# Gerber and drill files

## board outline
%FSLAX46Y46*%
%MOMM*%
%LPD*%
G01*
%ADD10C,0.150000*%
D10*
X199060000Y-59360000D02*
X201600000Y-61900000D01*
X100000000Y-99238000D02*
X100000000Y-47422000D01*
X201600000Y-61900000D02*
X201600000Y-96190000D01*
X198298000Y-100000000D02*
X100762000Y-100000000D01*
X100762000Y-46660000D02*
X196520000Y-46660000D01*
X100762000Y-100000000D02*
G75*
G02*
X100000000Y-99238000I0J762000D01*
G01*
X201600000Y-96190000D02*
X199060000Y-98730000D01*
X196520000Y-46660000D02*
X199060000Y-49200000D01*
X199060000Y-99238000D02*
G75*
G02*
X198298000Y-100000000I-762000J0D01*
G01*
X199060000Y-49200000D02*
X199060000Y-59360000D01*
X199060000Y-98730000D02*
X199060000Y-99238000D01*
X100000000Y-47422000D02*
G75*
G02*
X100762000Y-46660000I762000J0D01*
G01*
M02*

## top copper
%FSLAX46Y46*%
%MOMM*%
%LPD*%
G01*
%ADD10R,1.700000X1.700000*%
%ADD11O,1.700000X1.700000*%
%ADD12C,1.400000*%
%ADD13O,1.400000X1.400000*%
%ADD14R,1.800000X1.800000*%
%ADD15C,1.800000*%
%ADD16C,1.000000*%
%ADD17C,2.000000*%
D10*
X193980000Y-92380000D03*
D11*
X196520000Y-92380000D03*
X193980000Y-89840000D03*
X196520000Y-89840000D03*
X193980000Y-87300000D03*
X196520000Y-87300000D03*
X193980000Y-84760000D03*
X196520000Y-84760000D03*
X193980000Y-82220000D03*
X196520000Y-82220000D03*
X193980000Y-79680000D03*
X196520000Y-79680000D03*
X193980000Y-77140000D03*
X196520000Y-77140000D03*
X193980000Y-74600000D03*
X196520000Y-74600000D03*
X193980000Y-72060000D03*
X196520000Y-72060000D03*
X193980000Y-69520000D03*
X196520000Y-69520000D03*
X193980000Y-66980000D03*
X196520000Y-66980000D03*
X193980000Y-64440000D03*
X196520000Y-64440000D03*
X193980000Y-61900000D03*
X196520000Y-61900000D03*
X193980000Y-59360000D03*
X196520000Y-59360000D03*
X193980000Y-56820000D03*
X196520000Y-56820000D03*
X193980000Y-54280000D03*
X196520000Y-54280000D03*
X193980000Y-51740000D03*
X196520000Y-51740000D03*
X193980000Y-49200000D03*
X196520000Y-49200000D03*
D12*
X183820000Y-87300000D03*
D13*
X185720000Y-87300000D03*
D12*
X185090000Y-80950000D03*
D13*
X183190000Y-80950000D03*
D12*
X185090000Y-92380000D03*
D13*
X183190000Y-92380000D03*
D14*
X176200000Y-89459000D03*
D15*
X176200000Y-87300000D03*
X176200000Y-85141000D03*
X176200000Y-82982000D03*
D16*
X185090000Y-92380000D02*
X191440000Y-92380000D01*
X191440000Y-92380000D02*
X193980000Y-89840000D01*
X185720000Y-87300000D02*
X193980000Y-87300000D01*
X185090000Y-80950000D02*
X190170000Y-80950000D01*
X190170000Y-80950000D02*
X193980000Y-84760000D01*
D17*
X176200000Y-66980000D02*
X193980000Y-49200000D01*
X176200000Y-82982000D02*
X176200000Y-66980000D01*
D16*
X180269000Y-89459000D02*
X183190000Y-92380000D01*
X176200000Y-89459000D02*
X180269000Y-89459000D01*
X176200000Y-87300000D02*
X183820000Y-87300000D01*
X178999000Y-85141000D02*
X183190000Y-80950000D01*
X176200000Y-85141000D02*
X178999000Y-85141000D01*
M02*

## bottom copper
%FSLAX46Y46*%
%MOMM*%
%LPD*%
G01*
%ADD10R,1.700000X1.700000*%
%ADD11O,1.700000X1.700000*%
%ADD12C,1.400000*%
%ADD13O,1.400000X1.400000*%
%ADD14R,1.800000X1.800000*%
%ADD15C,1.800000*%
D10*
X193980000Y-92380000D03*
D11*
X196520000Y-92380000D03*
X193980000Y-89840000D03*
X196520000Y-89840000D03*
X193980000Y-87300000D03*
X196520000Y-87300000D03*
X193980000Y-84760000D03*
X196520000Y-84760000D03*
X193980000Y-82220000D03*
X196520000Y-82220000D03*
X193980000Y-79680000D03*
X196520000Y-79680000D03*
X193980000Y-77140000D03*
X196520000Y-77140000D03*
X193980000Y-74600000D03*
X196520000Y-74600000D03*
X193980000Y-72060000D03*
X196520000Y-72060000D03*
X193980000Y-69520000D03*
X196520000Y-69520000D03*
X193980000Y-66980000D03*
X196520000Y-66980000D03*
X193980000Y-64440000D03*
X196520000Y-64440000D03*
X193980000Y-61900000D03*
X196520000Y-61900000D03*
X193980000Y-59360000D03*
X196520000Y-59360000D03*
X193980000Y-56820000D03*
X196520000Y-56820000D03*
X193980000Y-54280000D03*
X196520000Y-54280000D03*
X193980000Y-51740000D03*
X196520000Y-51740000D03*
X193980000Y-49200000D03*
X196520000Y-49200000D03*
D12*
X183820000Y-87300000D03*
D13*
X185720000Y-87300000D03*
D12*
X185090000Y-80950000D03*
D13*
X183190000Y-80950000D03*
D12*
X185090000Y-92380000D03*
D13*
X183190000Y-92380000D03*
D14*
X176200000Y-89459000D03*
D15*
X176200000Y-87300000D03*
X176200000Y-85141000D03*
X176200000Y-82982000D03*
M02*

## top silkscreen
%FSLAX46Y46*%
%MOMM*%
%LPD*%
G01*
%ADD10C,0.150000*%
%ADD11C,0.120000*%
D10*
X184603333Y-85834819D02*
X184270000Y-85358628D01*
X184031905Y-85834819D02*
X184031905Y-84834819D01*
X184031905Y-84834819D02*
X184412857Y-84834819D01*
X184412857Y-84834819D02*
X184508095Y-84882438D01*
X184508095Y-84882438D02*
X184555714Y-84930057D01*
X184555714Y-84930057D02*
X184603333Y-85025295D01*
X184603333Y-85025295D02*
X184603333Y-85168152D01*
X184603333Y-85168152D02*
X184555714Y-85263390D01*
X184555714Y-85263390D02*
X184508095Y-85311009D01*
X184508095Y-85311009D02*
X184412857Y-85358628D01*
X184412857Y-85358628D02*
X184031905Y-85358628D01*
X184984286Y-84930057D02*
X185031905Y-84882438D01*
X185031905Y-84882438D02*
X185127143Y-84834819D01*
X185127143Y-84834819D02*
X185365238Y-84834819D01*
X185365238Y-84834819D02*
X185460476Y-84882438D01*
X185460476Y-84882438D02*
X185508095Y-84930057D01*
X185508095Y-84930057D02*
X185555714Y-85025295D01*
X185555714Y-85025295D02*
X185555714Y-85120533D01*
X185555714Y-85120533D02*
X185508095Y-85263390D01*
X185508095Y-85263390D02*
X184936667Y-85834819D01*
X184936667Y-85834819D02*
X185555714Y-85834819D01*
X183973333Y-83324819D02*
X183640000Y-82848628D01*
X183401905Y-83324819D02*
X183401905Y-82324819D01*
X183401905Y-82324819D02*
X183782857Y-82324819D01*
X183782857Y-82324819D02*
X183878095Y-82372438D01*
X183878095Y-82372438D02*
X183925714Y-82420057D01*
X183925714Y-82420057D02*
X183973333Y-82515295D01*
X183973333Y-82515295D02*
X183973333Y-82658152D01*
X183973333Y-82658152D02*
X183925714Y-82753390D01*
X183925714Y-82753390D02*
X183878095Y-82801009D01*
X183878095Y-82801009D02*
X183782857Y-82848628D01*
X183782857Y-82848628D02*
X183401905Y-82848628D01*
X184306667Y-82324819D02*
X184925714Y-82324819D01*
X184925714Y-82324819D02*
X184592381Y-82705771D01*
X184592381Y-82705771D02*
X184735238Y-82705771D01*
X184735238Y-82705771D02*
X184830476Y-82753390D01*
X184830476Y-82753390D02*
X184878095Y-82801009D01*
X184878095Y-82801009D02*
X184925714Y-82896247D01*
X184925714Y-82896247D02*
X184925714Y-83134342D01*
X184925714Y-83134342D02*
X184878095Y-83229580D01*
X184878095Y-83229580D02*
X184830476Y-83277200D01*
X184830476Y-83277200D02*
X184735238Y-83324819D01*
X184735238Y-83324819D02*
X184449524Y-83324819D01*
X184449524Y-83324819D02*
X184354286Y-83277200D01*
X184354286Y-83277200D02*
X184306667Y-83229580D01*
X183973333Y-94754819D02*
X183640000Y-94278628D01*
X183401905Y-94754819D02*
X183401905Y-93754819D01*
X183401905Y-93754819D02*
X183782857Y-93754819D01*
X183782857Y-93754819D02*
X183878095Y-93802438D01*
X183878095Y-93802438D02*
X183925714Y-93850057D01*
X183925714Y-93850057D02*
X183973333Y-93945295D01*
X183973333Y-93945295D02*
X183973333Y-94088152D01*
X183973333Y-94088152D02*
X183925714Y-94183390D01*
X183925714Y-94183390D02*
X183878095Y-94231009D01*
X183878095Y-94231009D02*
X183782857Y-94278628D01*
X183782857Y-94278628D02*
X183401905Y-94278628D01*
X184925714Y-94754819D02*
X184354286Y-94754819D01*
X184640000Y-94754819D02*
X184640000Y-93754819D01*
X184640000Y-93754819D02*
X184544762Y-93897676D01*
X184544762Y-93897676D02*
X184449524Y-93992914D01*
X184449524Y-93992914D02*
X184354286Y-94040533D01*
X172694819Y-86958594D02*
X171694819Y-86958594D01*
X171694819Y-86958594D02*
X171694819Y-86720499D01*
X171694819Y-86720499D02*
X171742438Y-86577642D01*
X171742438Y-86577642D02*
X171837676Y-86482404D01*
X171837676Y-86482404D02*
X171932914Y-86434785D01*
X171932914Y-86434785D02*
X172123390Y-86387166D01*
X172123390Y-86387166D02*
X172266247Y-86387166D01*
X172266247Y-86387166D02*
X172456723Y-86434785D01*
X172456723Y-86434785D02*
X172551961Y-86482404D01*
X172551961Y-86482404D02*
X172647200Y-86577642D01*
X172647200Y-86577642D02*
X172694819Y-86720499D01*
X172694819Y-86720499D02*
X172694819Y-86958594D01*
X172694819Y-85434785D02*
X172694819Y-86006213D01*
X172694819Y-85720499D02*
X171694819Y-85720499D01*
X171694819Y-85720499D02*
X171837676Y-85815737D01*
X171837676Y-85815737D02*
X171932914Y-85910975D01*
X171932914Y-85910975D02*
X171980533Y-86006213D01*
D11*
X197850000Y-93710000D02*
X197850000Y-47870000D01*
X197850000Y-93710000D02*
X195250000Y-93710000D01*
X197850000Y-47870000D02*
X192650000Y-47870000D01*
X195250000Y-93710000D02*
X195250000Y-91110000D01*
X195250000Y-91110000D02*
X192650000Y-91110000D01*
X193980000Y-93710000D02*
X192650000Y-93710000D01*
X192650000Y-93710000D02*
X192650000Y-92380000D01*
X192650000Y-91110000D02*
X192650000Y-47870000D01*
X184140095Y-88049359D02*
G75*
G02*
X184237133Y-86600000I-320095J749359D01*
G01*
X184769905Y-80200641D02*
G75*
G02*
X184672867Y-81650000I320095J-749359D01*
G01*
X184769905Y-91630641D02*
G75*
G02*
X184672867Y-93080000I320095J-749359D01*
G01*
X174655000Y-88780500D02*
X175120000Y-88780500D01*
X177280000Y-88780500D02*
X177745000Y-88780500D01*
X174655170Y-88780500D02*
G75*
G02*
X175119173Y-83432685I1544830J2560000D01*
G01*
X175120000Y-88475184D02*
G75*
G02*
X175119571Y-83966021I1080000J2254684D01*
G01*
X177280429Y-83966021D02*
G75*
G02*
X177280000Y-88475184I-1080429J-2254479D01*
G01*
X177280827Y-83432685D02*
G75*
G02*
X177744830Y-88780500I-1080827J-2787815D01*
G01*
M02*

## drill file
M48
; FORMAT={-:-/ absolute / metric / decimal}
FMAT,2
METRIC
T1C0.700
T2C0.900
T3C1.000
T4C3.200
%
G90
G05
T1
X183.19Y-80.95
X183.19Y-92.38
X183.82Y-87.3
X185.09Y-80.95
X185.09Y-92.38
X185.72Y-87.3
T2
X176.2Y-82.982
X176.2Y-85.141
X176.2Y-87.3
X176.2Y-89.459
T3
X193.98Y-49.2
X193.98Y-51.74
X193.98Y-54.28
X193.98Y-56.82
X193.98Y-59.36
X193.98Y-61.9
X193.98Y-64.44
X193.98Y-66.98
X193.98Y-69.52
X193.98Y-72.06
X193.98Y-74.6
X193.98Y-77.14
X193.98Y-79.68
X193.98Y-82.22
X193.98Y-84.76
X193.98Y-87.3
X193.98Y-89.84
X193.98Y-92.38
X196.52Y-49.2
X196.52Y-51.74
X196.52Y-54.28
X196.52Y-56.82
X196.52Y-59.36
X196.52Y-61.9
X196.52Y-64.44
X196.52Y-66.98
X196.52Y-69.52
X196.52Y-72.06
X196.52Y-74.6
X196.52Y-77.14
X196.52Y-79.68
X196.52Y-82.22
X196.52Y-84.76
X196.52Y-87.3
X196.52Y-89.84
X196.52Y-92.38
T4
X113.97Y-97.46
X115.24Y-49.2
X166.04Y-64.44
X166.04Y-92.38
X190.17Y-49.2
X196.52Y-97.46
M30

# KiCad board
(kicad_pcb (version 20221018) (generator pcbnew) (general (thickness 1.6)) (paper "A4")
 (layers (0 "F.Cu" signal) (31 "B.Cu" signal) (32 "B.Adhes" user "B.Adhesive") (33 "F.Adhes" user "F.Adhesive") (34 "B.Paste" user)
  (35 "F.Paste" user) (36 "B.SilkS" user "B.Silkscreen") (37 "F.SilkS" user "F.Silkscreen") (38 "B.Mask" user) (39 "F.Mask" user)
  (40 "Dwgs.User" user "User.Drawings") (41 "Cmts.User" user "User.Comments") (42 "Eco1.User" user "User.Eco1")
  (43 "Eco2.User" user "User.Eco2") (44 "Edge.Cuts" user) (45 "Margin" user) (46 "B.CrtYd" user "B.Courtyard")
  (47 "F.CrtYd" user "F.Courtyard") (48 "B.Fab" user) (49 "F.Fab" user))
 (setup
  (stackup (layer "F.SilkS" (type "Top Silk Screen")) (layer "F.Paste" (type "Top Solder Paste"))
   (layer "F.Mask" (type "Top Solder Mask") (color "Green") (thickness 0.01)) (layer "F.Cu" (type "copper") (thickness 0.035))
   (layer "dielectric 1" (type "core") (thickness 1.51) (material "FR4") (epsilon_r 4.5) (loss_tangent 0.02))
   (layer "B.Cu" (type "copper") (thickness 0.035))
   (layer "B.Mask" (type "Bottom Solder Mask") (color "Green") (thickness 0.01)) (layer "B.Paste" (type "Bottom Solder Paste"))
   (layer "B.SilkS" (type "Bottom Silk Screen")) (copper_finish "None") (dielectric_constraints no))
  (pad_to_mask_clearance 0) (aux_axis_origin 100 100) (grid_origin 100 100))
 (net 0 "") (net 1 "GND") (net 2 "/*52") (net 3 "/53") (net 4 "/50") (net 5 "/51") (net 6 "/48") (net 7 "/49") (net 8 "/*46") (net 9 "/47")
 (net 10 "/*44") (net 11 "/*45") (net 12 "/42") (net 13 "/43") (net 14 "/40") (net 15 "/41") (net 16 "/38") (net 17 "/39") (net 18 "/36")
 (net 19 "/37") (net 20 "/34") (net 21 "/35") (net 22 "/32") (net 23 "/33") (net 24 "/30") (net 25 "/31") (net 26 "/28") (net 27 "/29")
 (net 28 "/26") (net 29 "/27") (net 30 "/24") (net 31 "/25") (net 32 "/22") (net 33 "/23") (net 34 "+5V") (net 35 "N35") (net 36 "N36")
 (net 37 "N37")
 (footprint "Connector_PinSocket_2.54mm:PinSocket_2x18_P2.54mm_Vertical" (layer "F.Cu") (at 193.98 92.38 180)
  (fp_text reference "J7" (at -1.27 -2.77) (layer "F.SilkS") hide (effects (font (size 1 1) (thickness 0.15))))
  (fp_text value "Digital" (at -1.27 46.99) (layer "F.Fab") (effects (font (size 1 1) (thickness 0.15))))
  (fp_line (start -3.87 -1.33) (end -3.87 44.51) (stroke (width 0.12) (type solid)) (layer "F.SilkS"))
  (fp_line (start -3.87 -1.33) (end -1.27 -1.33) (stroke (width 0.12) (type solid)) (layer "F.SilkS"))
  (fp_line (start -3.87 44.51) (end 1.33 44.51) (stroke (width 0.12) (type solid)) (layer "F.SilkS"))
  (fp_line (start -1.27 -1.33) (end -1.27 1.27) (stroke (width 0.12) (type solid)) (layer "F.SilkS"))
  (fp_line (start -1.27 1.27) (end 1.33 1.27) (stroke (width 0.12) (type solid)) (layer "F.SilkS"))
  (fp_line (start 0 -1.33) (end 1.33 -1.33) (stroke (width 0.12) (type solid)) (layer "F.SilkS"))
  (fp_line (start 1.33 -1.33) (end 1.33 0) (stroke (width 0.12) (type solid)) (layer "F.SilkS"))
  (fp_line (start 1.33 1.27) (end 1.33 44.51) (stroke (width 0.12) (type solid)) (layer "F.SilkS"))
  (pad "1" thru_hole rect (at 0 0 180) (size 1.7 1.7) (drill 1) (layers "*.Cu" "*.Mask") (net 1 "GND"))
  (pad "2" thru_hole oval (at -2.54 0 180) (size 1.7 1.7) (drill 1) (layers "*.Cu" "*.Mask") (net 1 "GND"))
  (pad "3" thru_hole oval (at 0 2.54 180) (size 1.7 1.7) (drill 1) (layers "*.Cu" "*.Mask") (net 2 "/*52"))
  (pad "4" thru_hole oval (at -2.54 2.54 180) (size 1.7 1.7) (drill 1) (layers "*.Cu" "*.Mask") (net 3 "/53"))
  (pad "5" thru_hole oval (at 0 5.08 180) (size 1.7 1.7) (drill 1) (layers "*.Cu" "*.Mask") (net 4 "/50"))
  (pad "6" thru_hole oval (at -2.54 5.08 180) (size 1.7 1.7) (drill 1) (layers "*.Cu" "*.Mask") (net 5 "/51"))
  (pad "7" thru_hole oval (at 0 7.62 180) (size 1.7 1.7) (drill 1) (layers "*.Cu" "*.Mask") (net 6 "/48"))
  (pad "8" thru_hole oval (at -2.54 7.62 180) (size 1.7 1.7) (drill 1) (layers "*.Cu" "*.Mask") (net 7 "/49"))
  (pad "9" thru_hole oval (at 0 10.16 180) (size 1.7 1.7) (drill 1) (layers "*.Cu" "*.Mask") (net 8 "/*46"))
  (pad "10" thru_hole oval (at -2.54 10.16 180) (size 1.7 1.7) (drill 1) (layers "*.Cu" "*.Mask") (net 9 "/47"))
  (pad "11" thru_hole oval (at 0 12.7 180) (size 1.7 1.7) (drill 1) (layers "*.Cu" "*.Mask") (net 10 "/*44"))
  (pad "12" thru_hole oval (at -2.54 12.7 180) (size 1.7 1.7) (drill 1) (layers "*.Cu" "*.Mask") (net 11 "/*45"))
  (pad "13" thru_hole oval (at 0 15.24 180) (size 1.7 1.7) (drill 1) (layers "*.Cu" "*.Mask") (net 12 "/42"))
  (pad "14" thru_hole oval (at -2.54 15.24 180) (size 1.7 1.7) (drill 1) (layers "*.Cu" "*.Mask") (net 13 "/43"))
  (pad "15" thru_hole oval (at 0 17.78 180) (size 1.7 1.7) (drill 1) (layers "*.Cu" "*.Mask") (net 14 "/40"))
  (pad "16" thru_hole oval (at -2.54 17.78 180) (size 1.7 1.7) (drill 1) (layers "*.Cu" "*.Mask") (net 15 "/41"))
  (pad "17" thru_hole oval (at 0 20.32 180) (size 1.7 1.7) (drill 1) (layers "*.Cu" "*.Mask") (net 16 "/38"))
  (pad "18" thru_hole oval (at -2.54 20.32 180) (size 1.7 1.7) (drill 1) (layers "*.Cu" "*.Mask") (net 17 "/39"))
  (pad "19" thru_hole oval (at 0 22.86 180) (size 1.7 1.7) (drill 1) (layers "*.Cu" "*.Mask") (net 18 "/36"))
  (pad "20" thru_hole oval (at -2.54 22.86 180) (size 1.7 1.7) (drill 1) (layers "*.Cu" "*.Mask") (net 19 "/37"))
  (pad "21" thru_hole oval (at 0 25.4 180) (size 1.7 1.7) (drill 1) (layers "*.Cu" "*.Mask") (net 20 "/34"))
  (pad "22" thru_hole oval (at -2.54 25.4 180) (size 1.7 1.7) (drill 1) (layers "*.Cu" "*.Mask") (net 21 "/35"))
  (pad "23" thru_hole oval (at 0 27.94 180) (size 1.7 1.7) (drill 1) (layers "*.Cu" "*.Mask") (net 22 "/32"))
  (pad "24" thru_hole oval (at -2.54 27.94 180) (size 1.7 1.7) (drill 1) (layers "*.Cu" "*.Mask") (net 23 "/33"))
  (pad "25" thru_hole oval (at 0 30.48 180) (size 1.7 1.7) (drill 1) (layers "*.Cu" "*.Mask") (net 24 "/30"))
  (pad "26" thru_hole oval (at -2.54 30.48 180) (size 1.7 1.7) (drill 1) (layers "*.Cu" "*.Mask") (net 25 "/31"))
  (pad "27" thru_hole oval (at 0 33.02 180) (size 1.7 1.7) (drill 1) (layers "*.Cu" "*.Mask") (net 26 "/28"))
  (pad "28" thru_hole oval (at -2.54 33.02 180) (size 1.7 1.7) (drill 1) (layers "*.Cu" "*.Mask") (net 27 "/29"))
  (pad "29" thru_hole oval (at 0 35.56 180) (size 1.7 1.7) (drill 1) (layers "*.Cu" "*.Mask") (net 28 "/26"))
  (pad "30" thru_hole oval (at -2.54 35.56 180) (size 1.7 1.7) (drill 1) (layers "*.Cu" "*.Mask") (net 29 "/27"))
  (pad "31" thru_hole oval (at 0 38.1 180) (size 1.7 1.7) (drill 1) (layers "*.Cu" "*.Mask") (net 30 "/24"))
  (pad "32" thru_hole oval (at -2.54 38.1 180) (size 1.7 1.7) (drill 1) (layers "*.Cu" "*.Mask") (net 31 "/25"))
  (pad "33" thru_hole oval (at 0 40.64 180) (size 1.7 1.7) (drill 1) (layers "*.Cu" "*.Mask") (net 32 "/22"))
  (pad "34" thru_hole oval (at -2.54 40.64 180) (size 1.7 1.7) (drill 1) (layers "*.Cu" "*.Mask") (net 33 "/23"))
  (pad "35" thru_hole oval (at 0 43.18 180) (size 1.7 1.7) (drill 1) (layers "*.Cu" "*.Mask") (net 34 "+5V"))
  (pad "36" thru_hole oval (at -2.54 43.18 180) (size 1.7 1.7) (drill 1) (layers "*.Cu" "*.Mask") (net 34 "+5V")))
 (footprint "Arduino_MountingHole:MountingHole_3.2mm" (layer "F.Cu") (at 196.52 97.46)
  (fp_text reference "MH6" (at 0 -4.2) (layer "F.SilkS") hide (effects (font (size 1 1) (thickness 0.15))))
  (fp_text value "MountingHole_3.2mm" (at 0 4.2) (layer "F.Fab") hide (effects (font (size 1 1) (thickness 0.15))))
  (pad "" np_thru_hole circle (at 0 0) (size 3.2 3.2) (drill 3.2) (layers "*.Cu" "*.Mask")))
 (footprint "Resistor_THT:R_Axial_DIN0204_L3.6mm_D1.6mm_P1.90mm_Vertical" (layer "F.Cu") (at 183.82 87.3)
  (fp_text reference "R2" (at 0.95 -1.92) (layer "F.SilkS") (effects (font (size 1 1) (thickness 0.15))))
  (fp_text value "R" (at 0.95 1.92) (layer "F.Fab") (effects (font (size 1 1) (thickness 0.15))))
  (fp_arc (start 0.320095 0.749359) (mid -0.813042 -0.054435) (end 0.417133 -0.7) (stroke (width 0.12) (type solid)) (layer "F.SilkS"))
  (pad "1" thru_hole circle (at 0 0) (size 1.4 1.4) (drill 0.7) (layers "*.Cu" "*.Mask") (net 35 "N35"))
  (pad "2" thru_hole oval (at 1.9 0) (size 1.4 1.4) (drill 0.7) (layers "*.Cu" "*.Mask") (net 4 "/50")))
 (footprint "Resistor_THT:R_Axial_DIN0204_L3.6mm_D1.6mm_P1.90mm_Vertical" (layer "F.Cu") (at 185.09 80.95 180)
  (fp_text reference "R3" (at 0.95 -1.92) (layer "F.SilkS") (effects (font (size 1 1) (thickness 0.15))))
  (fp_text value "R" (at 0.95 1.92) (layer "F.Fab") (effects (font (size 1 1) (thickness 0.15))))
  (fp_arc (start 0.320095 0.749359) (mid -0.813042 -0.054435) (end 0.417133 -0.7) (stroke (width 0.12) (type solid)) (layer "F.SilkS"))
  (pad "1" thru_hole circle (at 0 0 180) (size 1.4 1.4) (drill 0.7) (layers "*.Cu" "*.Mask") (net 6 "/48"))
  (pad "2" thru_hole oval (at 1.9 0 180) (size 1.4 1.4) (drill 0.7) (layers "*.Cu" "*.Mask") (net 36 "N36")))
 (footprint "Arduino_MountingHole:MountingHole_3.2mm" (layer "F.Cu") (at 115.24 49.2)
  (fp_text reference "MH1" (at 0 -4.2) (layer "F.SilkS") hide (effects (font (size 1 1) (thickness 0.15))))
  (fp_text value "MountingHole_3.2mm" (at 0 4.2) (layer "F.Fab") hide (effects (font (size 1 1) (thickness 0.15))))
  (pad "" np_thru_hole circle (at 0 0) (size 3.2 3.2) (drill 3.2) (layers "*.Cu" "*.Mask")))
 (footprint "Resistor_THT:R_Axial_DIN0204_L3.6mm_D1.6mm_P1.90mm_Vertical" (layer "F.Cu") (at 185.09 92.38 180)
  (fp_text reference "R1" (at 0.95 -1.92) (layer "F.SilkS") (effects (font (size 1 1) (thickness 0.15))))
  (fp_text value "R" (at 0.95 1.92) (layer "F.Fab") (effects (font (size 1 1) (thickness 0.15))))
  (fp_arc (start 0.320095 0.749359) (mid -0.813042 -0.054435) (end 0.417133 -0.7) (stroke (width 0.12) (type solid)) (layer "F.SilkS"))
  (pad "1" thru_hole circle (at 0 0 180) (size 1.4 1.4) (drill 0.7) (layers "*.Cu" "*.Mask") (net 2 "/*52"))
  (pad "2" thru_hole oval (at 1.9 0 180) (size 1.4 1.4) (drill 0.7) (layers "*.Cu" "*.Mask") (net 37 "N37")))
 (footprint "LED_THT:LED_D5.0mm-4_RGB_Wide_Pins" (layer "F.Cu") (at 176.2 89.459 90)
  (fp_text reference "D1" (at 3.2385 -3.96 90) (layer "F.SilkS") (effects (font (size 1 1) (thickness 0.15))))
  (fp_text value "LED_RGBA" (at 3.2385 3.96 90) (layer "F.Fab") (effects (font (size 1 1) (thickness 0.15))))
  (fp_line (start 0.6785 -1.545) (end 0.6785 -1.08) (stroke (width 0.12) (type solid)) (layer "F.SilkS"))
  (fp_line (start 0.6785 1.08) (end 0.6785 1.545) (stroke (width 0.12) (type solid)) (layer "F.SilkS"))
  (fp_arc (start 0.6785 -1.54483) (mid 3.496956 -2.978809) (end 6.026315 -1.080827) (stroke (width 0.12) (type solid)) (layer "F.SilkS"))
  (fp_arc (start 0.983816 -1.08) (mid 3.238262 -2.5) (end 5.492979 -1.080429) (stroke (width 0.12) (type solid)) (layer "F.SilkS"))
  (fp_arc (start 5.492979 1.080429) (mid 3.238262 2.5) (end 0.983816 1.08) (stroke (width 0.12) (type solid)) (layer "F.SilkS"))
  (fp_arc (start 6.026315 1.080827) (mid 3.496956 2.978808) (end 0.6785 1.54483) (stroke (width 0.12) (type solid)) (layer "F.SilkS"))
  (pad "1" thru_hole rect (at 0 0 90) (size 1.8 1.8) (drill 0.9) (layers "*.Cu" "*.Mask") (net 37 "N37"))
  (pad "2" thru_hole circle (at 2.159 0 90) (size 1.8 1.8) (drill 0.9) (layers "*.Cu" "*.Mask") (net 35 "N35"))
  (pad "3" thru_hole circle (at 4.318 0 90) (size 1.8 1.8) (drill 0.9) (layers "*.Cu" "*.Mask") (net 36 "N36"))
  (pad "4" thru_hole circle (at 6.477 0 90) (size 1.8 1.8) (drill 0.9) (layers "*.Cu" "*.Mask") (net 34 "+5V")))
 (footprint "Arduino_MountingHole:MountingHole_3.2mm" (layer "F.Cu") (at 113.97 97.46)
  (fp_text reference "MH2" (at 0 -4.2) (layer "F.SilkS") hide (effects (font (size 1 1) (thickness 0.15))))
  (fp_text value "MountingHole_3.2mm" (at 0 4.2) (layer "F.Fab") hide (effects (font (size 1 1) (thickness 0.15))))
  (pad "" np_thru_hole circle (at 0 0) (size 3.2 3.2) (drill 3.2) (layers "*.Cu" "*.Mask")))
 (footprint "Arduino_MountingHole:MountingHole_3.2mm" (layer "F.Cu") (at 166.04 64.44)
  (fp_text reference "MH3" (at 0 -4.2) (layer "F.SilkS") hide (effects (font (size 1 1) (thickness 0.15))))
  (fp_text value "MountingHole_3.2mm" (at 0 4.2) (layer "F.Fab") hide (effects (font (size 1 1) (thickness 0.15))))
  (pad "" np_thru_hole circle (at 0 0) (size 3.2 3.2) (drill 3.2) (layers "*.Cu" "*.Mask")))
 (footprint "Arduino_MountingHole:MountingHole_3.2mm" (layer "F.Cu") (at 166.04 92.38)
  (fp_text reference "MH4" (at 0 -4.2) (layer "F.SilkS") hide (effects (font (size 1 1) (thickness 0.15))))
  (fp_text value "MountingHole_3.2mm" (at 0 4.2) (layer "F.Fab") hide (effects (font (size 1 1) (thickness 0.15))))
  (pad "" np_thru_hole circle (at 0 0) (size 3.2 3.2) (drill 3.2) (layers "*.Cu" "*.Mask")))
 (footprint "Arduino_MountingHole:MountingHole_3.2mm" (layer "F.Cu") (at 190.17 49.2)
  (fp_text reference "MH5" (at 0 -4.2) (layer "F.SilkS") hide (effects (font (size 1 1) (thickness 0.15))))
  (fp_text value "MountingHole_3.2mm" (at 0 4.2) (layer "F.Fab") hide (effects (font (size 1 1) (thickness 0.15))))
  (pad "" np_thru_hole circle (at 0 0) (size 3.2 3.2) (drill 3.2) (layers "*.Cu" "*.Mask")))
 (gr_line (start 199.06 59.36) (end 201.6 61.9) (stroke (width 0.15) (type solid)) (layer "Edge.Cuts"))
 (gr_line (start 100 99.238) (end 100 47.422) (stroke (width 0.15) (type solid)) (layer "Edge.Cuts"))
 (gr_line (start 201.6 61.9) (end 201.6 96.19) (stroke (width 0.15) (type solid)) (layer "Edge.Cuts"))
 (gr_line (start 198.298 100) (end 100.762 100) (stroke (width 0.15) (type solid)) (layer "Edge.Cuts"))
 (gr_line (start 100.762 46.66) (end 196.52 46.66) (stroke (width 0.15) (type solid)) (layer "Edge.Cuts"))
 (gr_arc (start 100.762 100) (mid 100.223185 99.776815) (end 100 99.238) (stroke (width 0.15) (type solid)) (layer "Edge.Cuts"))
 (gr_line (start 201.6 96.19) (end 199.06 98.73) (stroke (width 0.15) (type solid)) (layer "Edge.Cuts"))
 (gr_line (start 196.52 46.66) (end 199.06 49.2) (stroke (width 0.15) (type solid)) (layer "Edge.Cuts"))
 (gr_arc (start 199.06 99.238) (mid 198.836815 99.776815) (end 198.298 100) (stroke (width 0.15) (type solid)) (layer "Edge.Cuts"))
 (gr_line (start 199.06 49.2) (end 199.06 59.36) (stroke (width 0.15) (type solid)) (layer "Edge.Cuts"))
 (gr_line (start 199.06 98.73) (end 199.06 99.238) (stroke (width 0.15) (type solid)) (layer "Edge.Cuts"))
 (gr_arc (start 100 47.422) (mid 100.223185 46.883185) (end 100.762 46.66) (stroke (width 0.15) (type solid)) (layer "Edge.Cuts"))
 (segment (start 185.09 92.38) (end 191.44 92.38) (width 1) (layer "F.Cu") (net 2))
 (segment (start 191.44 92.38) (end 193.98 89.84) (width 1) (layer "F.Cu") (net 2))
 (segment (start 185.72 87.3) (end 193.98 87.3) (width 1) (layer "F.Cu") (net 4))
 (segment (start 185.09 80.95) (end 190.17 80.95) (width 1) (layer "F.Cu") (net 6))
 (segment (start 190.17 80.95) (end 193.98 84.76) (width 1) (layer "F.Cu") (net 6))
 (segment (start 176.2 66.98) (end 193.98 49.2) (width 2) (layer "F.Cu") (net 34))
 (segment (start 176.2 82.982) (end 176.2 66.98) (width 2) (layer "F.Cu") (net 34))
 (segment (start 180.269 89.459) (end 183.19 92.38) (width 1) (layer "F.Cu") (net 37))
 (segment (start 176.2 89.459) (end 180.269 89.459) (width 1) (layer "F.Cu") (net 37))
 (segment (start 176.2 87.3) (end 183.82 87.3) (width 1) (layer "F.Cu") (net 35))
 (segment (start 178.999 85.141) (end 183.19 80.95) (width 1) (layer "F.Cu") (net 36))
 (segment (start 176.2 85.141) (end 178.999 85.141) (width 1) (layer "F.Cu") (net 36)))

